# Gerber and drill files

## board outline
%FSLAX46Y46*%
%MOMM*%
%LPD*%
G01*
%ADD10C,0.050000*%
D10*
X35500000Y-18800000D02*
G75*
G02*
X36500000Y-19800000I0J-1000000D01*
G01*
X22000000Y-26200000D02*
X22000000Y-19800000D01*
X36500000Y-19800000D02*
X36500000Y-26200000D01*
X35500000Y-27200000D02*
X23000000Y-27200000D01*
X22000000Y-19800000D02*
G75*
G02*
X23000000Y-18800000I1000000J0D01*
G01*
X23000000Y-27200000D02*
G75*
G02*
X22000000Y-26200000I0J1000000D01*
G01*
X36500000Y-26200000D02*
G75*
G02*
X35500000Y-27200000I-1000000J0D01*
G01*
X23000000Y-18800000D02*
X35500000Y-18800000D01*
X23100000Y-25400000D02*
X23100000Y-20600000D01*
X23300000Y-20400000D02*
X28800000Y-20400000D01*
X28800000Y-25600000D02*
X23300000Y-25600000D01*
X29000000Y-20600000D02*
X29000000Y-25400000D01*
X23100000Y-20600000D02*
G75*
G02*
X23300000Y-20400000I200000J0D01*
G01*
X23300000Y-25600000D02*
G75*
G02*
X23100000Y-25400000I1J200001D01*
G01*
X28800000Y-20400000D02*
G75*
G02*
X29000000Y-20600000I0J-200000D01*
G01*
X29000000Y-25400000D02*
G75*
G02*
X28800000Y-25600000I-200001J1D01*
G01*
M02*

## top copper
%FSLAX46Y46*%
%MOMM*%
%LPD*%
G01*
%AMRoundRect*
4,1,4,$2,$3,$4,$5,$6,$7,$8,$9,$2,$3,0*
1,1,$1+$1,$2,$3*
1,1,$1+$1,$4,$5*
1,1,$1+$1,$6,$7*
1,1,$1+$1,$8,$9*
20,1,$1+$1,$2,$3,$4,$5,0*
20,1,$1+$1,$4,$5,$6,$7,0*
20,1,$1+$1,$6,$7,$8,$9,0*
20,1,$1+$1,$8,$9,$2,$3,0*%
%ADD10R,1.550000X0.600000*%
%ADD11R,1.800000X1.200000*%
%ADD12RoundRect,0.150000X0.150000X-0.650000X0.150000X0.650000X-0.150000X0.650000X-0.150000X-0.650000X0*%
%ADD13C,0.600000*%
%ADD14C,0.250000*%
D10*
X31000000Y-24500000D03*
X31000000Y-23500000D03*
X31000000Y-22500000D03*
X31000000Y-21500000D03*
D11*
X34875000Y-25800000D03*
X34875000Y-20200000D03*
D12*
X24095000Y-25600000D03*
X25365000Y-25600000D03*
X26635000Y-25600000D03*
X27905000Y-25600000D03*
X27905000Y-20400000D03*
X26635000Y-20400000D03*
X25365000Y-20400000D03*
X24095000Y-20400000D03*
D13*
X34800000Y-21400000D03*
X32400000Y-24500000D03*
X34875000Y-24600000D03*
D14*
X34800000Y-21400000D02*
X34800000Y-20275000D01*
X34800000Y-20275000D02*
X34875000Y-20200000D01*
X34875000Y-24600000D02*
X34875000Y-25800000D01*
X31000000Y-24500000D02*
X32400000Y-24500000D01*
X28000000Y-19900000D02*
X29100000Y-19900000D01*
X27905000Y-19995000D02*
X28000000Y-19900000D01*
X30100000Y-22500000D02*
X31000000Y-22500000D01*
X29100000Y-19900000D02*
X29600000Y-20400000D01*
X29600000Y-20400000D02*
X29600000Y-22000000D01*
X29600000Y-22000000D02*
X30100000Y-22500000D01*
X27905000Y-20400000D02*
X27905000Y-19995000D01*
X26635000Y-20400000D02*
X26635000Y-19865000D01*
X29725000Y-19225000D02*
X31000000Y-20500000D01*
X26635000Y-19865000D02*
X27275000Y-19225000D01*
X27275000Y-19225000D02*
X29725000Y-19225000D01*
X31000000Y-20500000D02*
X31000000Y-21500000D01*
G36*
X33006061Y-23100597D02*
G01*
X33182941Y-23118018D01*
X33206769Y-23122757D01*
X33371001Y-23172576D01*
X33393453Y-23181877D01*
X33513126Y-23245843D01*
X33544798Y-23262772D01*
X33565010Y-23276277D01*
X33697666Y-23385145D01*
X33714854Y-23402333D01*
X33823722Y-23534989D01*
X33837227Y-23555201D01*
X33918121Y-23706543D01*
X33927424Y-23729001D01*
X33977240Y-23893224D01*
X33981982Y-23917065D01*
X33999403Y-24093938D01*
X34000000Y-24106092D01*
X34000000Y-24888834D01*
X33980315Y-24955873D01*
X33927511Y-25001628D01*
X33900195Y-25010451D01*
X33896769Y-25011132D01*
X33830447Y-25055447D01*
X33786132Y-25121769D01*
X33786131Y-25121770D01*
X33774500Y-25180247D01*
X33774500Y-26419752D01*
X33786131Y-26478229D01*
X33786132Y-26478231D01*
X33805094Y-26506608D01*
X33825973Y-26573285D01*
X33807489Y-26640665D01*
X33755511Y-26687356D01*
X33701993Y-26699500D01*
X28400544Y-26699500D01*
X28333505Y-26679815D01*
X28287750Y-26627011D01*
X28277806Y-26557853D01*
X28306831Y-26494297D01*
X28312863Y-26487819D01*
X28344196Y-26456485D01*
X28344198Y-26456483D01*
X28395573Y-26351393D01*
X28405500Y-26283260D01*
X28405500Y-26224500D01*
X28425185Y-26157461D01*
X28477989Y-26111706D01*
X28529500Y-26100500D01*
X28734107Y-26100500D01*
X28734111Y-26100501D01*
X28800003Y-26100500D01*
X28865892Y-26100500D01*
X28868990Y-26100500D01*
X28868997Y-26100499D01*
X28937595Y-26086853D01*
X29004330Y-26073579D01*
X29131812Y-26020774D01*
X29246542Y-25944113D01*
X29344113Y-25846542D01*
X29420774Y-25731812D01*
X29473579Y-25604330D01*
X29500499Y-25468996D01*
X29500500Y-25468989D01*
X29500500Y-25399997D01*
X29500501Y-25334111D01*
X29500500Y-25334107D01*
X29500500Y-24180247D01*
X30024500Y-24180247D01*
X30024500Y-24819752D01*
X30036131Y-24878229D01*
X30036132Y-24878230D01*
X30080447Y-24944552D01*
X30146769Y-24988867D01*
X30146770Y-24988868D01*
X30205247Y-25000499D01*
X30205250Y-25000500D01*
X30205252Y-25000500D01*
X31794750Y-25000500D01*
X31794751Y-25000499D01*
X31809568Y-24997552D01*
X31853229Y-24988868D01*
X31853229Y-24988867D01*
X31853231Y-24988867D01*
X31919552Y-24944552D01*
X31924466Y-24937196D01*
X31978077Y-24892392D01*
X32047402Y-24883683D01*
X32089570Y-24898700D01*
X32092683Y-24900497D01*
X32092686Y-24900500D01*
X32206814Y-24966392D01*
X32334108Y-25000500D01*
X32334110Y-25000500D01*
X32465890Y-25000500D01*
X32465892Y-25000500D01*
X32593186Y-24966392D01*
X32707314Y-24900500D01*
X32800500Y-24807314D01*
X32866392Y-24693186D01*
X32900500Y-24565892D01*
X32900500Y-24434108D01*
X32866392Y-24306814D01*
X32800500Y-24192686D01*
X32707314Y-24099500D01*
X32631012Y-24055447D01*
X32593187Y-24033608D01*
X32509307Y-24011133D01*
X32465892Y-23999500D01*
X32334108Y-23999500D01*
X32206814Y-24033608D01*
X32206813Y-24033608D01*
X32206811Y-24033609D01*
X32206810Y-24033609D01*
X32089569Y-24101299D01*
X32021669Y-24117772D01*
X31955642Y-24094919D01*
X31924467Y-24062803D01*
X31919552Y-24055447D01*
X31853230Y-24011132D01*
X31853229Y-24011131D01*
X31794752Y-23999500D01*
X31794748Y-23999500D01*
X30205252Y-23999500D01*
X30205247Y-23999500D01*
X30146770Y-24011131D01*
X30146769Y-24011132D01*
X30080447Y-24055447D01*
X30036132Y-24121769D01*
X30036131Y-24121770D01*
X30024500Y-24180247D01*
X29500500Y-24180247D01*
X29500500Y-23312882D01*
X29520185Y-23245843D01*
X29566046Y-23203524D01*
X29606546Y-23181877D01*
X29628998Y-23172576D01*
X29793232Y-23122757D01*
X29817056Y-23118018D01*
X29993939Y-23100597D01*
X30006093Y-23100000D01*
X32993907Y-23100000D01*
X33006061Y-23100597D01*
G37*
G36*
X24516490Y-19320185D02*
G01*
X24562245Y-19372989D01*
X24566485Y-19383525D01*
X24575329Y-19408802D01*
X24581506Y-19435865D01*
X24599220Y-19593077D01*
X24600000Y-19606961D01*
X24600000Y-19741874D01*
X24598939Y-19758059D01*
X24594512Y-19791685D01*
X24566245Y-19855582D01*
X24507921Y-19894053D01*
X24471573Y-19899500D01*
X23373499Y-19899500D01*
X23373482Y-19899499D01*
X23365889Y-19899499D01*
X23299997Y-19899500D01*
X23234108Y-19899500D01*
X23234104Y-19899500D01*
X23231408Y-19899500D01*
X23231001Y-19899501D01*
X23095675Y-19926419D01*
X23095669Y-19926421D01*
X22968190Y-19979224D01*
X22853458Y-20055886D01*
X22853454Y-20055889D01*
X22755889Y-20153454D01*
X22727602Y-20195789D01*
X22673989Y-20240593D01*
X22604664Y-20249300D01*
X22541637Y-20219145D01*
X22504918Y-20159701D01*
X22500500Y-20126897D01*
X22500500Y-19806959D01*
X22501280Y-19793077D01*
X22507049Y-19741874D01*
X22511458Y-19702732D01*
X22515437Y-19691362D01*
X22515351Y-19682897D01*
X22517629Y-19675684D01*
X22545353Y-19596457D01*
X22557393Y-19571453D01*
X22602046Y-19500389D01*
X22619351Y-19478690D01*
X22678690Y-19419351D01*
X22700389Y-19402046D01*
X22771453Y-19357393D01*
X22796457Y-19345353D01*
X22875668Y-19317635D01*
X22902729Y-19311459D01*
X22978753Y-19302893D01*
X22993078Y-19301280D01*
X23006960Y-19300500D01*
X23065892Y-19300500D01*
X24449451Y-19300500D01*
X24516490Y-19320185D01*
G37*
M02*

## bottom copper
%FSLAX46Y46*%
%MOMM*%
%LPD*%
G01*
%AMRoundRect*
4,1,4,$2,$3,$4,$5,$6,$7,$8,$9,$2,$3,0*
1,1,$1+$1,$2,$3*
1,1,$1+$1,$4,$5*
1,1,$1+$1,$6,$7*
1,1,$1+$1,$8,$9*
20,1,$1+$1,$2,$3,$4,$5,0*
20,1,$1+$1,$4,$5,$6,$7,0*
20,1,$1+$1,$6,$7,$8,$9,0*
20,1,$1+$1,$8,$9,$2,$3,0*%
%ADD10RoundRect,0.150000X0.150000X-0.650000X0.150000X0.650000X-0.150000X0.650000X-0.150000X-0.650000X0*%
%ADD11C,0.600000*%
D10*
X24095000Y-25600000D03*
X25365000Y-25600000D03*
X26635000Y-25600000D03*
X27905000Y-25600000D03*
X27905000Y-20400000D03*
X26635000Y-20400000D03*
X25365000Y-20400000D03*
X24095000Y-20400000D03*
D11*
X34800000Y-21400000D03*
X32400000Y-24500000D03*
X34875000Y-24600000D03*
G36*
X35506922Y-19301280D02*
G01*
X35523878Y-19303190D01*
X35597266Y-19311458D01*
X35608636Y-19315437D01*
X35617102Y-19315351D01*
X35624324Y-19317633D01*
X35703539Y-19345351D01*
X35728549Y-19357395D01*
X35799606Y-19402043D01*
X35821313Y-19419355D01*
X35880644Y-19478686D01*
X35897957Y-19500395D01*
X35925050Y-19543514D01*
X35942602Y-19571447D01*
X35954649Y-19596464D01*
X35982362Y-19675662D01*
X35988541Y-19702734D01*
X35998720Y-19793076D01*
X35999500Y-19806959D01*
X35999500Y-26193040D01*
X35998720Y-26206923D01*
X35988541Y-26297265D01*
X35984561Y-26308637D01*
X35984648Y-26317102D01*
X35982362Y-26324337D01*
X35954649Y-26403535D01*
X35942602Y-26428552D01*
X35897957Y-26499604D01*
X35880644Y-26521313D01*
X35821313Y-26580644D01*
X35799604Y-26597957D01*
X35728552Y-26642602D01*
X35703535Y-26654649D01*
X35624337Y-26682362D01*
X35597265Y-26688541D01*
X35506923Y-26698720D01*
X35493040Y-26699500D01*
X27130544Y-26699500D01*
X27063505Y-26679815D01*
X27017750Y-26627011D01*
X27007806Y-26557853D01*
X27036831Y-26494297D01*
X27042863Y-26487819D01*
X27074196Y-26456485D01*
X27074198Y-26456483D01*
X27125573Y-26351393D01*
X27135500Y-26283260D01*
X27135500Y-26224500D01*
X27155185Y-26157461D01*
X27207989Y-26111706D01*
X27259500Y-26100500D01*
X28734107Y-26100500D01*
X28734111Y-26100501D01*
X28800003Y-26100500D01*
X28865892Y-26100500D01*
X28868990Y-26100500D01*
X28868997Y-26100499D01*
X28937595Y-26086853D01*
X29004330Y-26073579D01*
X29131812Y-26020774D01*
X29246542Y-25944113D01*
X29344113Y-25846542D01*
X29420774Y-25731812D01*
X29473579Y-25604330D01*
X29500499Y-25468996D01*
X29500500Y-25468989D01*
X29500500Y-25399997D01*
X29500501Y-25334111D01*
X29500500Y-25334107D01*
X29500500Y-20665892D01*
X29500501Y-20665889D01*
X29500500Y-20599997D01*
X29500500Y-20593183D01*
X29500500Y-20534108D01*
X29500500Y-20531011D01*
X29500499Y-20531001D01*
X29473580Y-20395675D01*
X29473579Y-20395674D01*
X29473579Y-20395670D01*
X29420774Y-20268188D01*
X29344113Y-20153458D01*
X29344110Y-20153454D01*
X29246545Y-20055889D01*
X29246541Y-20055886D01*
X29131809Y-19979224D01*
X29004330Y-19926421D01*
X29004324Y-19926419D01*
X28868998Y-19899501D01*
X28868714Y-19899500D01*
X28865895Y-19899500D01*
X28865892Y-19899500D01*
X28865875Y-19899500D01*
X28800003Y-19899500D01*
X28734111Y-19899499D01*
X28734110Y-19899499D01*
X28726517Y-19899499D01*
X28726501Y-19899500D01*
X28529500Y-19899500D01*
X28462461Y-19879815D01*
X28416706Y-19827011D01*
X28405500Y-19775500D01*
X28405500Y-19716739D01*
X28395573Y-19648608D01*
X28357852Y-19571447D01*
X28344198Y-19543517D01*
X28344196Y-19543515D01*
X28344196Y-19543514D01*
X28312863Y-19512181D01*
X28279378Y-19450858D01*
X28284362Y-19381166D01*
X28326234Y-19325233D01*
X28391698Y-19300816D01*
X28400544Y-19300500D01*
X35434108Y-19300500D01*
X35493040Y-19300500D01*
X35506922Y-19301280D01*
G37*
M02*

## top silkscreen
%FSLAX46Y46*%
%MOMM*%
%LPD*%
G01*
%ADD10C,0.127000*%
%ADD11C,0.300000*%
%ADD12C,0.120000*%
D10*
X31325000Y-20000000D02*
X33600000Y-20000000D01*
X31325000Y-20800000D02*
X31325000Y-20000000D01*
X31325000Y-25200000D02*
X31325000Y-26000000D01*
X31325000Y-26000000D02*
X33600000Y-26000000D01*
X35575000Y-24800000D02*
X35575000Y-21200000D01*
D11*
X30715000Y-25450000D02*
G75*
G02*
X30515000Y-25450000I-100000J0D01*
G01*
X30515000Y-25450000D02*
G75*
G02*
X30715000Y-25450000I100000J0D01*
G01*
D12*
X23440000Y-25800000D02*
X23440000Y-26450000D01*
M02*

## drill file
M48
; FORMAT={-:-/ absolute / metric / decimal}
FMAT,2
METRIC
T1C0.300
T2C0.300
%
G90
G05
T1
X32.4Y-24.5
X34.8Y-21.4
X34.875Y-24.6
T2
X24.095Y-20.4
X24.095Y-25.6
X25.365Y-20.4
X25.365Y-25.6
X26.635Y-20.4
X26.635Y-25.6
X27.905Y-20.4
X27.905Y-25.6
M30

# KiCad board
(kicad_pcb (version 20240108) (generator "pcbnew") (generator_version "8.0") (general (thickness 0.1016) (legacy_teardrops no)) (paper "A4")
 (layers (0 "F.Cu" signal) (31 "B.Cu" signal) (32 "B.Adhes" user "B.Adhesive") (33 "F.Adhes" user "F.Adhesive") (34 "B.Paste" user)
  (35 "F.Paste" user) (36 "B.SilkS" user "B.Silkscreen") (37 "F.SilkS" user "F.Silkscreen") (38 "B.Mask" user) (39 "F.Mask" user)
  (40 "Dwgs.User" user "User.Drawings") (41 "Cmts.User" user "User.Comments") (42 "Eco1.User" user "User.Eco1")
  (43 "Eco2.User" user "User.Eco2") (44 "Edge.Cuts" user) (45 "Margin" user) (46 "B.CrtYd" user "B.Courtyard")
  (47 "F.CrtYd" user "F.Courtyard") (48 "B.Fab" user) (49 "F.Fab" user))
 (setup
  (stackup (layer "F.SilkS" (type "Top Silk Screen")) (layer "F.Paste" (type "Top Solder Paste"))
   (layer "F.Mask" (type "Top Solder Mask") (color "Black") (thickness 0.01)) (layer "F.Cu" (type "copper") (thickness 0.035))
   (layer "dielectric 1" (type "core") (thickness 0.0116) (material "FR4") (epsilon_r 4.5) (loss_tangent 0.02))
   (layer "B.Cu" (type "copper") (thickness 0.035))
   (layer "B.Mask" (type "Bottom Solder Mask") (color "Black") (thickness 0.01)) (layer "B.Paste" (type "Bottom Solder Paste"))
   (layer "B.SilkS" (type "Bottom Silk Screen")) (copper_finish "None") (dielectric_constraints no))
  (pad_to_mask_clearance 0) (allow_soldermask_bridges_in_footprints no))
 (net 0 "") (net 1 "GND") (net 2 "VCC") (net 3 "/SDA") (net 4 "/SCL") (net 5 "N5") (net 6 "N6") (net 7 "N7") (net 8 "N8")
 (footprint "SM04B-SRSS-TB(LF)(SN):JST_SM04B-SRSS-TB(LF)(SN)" (layer "F.Cu") (at 31 23 90)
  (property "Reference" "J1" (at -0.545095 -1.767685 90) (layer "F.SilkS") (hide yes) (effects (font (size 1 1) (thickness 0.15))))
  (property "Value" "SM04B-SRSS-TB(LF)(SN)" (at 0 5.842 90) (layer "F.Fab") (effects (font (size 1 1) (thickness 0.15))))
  (fp_line (start 3 0.325) (end 3 2.6) (stroke (width 0.127) (type solid)) (layer "F.SilkS"))
  (fp_line (start 2.2 0.325) (end 3 0.325) (stroke (width 0.127) (type solid)) (layer "F.SilkS"))
  (fp_line (start -2.2 0.325) (end -3 0.325) (stroke (width 0.127) (type solid)) (layer "F.SilkS"))
  (fp_line (start -3 0.325) (end -3 2.6) (stroke (width 0.127) (type solid)) (layer "F.SilkS"))
  (fp_line (start -1.8 4.575) (end 1.8 4.575) (stroke (width 0.127) (type solid)) (layer "F.SilkS"))
  (fp_circle (center -2.45 -0.385) (end -2.35 -0.385) (stroke (width 0.3) (type solid)) (fill none) (layer "F.SilkS"))
  (pad "1" smd rect (at -1.5 0 90) (size 0.6 1.55) (layers "F.Cu" "F.Paste" "F.Mask") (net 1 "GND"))
  (pad "2" smd rect (at -0.5 0 90) (size 0.6 1.55) (layers "F.Cu" "F.Paste" "F.Mask") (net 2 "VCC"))
  (pad "3" smd rect (at 0.5 0 90) (size 0.6 1.55) (layers "F.Cu" "F.Paste" "F.Mask") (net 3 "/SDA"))
  (pad "4" smd rect (at 1.5 0 90) (size 0.6 1.55) (layers "F.Cu" "F.Paste" "F.Mask") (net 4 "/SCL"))
  (pad "S1" smd rect (at -2.8 3.875 90) (size 1.2 1.8) (layers "F.Cu" "F.Paste" "F.Mask") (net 1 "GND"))
  (pad "S2" smd rect (at 2.8 3.875 90) (size 1.2 1.8) (layers "F.Cu" "F.Paste" "F.Mask") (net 1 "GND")))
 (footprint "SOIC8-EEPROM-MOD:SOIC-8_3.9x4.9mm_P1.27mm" (layer "F.Cu") (at 26 23 90)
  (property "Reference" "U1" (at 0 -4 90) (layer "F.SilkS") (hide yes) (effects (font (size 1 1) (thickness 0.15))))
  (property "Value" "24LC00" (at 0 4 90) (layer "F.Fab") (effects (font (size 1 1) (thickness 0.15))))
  (fp_line (start -2.8 -2.56) (end -3.45 -2.56) (stroke (width 0.12) (type solid)) (layer "F.SilkS"))
  (fp_line (start -2.4 -2.9) (end 2.4 -2.9) (stroke (width 0.05) (type default)) (layer "Edge.Cuts"))
  (fp_line (start 2.6 -2.7) (end 2.6 2.8) (stroke (width 0.05) (type default)) (layer "Edge.Cuts"))
  (fp_line (start -2.6 2.8) (end -2.6 -2.7) (stroke (width 0.05) (type default)) (layer "Edge.Cuts"))
  (fp_line (start 2.4 3) (end -2.4 3) (stroke (width 0.05) (type default)) (layer "Edge.Cuts"))
  (fp_arc (start 2.4 -2.9) (mid 2.541421 -2.841421) (end 2.6 -2.7) (stroke (width 0.05) (type default)) (layer "Edge.Cuts"))
  (fp_arc (start -2.6 -2.7) (mid -2.541421 -2.841421) (end -2.4 -2.9) (stroke (width 0.05) (type default)) (layer "Edge.Cuts"))
  (fp_arc (start 2.6 2.8) (mid 2.541421 2.941421) (end 2.4 3) (stroke (width 0.05) (type default)) (layer "Edge.Cuts"))
  (fp_arc (start -2.4 3) (mid -2.541421 2.941421) (end -2.6 2.8) (stroke (width 0.05) (type default)) (layer "Edge.Cuts"))
  (pad "1" thru_hole roundrect (at -2.6 -1.905 90) (size 1.6 0.6) (drill 0.3) (layers "*.Cu" "*.Mask") (remove_unused_layers no)
   (roundrect_rratio 0.25) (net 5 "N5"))
  (pad "2" thru_hole roundrect (at -2.6 -0.635 90) (size 1.6 0.6) (drill 0.3) (layers "*.Cu" "*.Mask") (remove_unused_layers no)
   (roundrect_rratio 0.25) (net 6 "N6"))
  (pad "3" thru_hole roundrect (at -2.6 0.635 90) (size 1.6 0.6) (drill 0.3) (layers "*.Cu" "*.Mask") (remove_unused_layers no)
   (roundrect_rratio 0.25) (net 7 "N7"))
  (pad "4" thru_hole roundrect (at -2.6 1.905 90) (size 1.6 0.6) (drill 0.3) (layers "*.Cu" "*.Mask") (remove_unused_layers no)
   (roundrect_rratio 0.25) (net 1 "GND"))
  (pad "5" thru_hole roundrect (at 2.6 1.905 90) (size 1.6 0.6) (drill 0.3) (layers "*.Cu" "*.Mask") (remove_unused_layers no)
   (roundrect_rratio 0.25) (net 3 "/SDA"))
  (pad "6" thru_hole roundrect (at 2.6 0.635 90) (size 1.6 0.6) (drill 0.3) (layers "*.Cu" "*.Mask") (remove_unused_layers no)
   (roundrect_rratio 0.25) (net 4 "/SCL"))
  (pad "7" thru_hole roundrect (at 2.6 -0.635 90) (size 1.6 0.6) (drill 0.3) (layers "*.Cu" "*.Mask") (remove_unused_layers no)
   (roundrect_rratio 0.25) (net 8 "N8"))
  (pad "8" thru_hole roundrect (at 2.6 -1.905 90) (size 1.6 0.6) (drill 0.3) (layers "*.Cu" "*.Mask") (remove_unused_layers no)
   (roundrect_rratio 0.25) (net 2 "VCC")))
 (gr_arc (start 35.5 18.8) (mid 36.207107 19.092893) (end 36.5 19.8) (stroke (width 0.05) (type default)) (layer "Edge.Cuts"))
 (gr_line (start 22 26.2) (end 22 19.8) (stroke (width 0.05) (type default)) (layer "Edge.Cuts"))
 (gr_line (start 36.5 19.8) (end 36.5 26.2) (stroke (width 0.05) (type default)) (layer "Edge.Cuts"))
 (gr_line (start 35.5 27.2) (end 23 27.2) (stroke (width 0.05) (type default)) (layer "Edge.Cuts"))
 (gr_arc (start 22 19.8) (mid 22.292893 19.092893) (end 23 18.8) (stroke (width 0.05) (type default)) (layer "Edge.Cuts"))
 (gr_arc (start 23 27.2) (mid 22.292893 26.907107) (end 22 26.2) (stroke (width 0.05) (type default)) (layer "Edge.Cuts"))
 (gr_arc (start 36.5 26.2) (mid 36.207107 26.907107) (end 35.5 27.2) (stroke (width 0.05) (type default)) (layer "Edge.Cuts"))
 (gr_line (start 23 18.8) (end 35.5 18.8) (stroke (width 0.05) (type default)) (layer "Edge.Cuts"))
 (segment (start 34.8 21.4) (end 34.8 20.275) (width 0.25) (layer "F.Cu") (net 1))
 (segment (start 34.8 20.275) (end 34.875 20.2) (width 0.25) (layer "F.Cu") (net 1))
 (segment (start 34.875 24.6) (end 34.875 25.8) (width 0.25) (layer "F.Cu") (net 1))
 (segment (start 31 24.5) (end 32.4 24.5) (width 0.25) (layer "F.Cu") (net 1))
 (via (at 34.8 21.4) (size 0.6) (drill 0.3) (layers "F.Cu" "B.Cu") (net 1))
 (via (at 32.4 24.5) (size 0.6) (drill 0.3) (layers "F.Cu" "B.Cu") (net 1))
 (via (at 34.875 24.6) (size 0.6) (drill 0.3) (layers "F.Cu" "B.Cu") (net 1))
 (segment (start 28 19.9) (end 29.1 19.9) (width 0.25) (layer "F.Cu") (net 3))
 (segment (start 27.905 19.995) (end 28 19.9) (width 0.25) (layer "F.Cu") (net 3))
 (segment (start 30.1 22.5) (end 31 22.5) (width 0.25) (layer "F.Cu") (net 3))
 (segment (start 29.1 19.9) (end 29.6 20.4) (width 0.25) (layer "F.Cu") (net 3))
 (segment (start 29.6 20.4) (end 29.6 22) (width 0.25) (layer "F.Cu") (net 3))
 (segment (start 29.6 22) (end 30.1 22.5) (width 0.25) (layer "F.Cu") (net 3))
 (segment (start 27.905 20.4) (end 27.905 19.995) (width 0.25) (layer "F.Cu") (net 3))
 (segment (start 26.635 20.4) (end 26.635 19.865) (width 0.25) (layer "F.Cu") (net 4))
 (segment (start 29.725 19.225) (end 31 20.5) (width 0.25) (layer "F.Cu") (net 4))
 (segment (start 26.635 19.865) (end 27.275 19.225) (width 0.25) (layer "F.Cu") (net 4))
 (segment (start 27.275 19.225) (end 29.725 19.225) (width 0.25) (layer "F.Cu") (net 4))
 (segment (start 31 20.5) (end 31 21.5) (width 0.25) (layer "F.Cu") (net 4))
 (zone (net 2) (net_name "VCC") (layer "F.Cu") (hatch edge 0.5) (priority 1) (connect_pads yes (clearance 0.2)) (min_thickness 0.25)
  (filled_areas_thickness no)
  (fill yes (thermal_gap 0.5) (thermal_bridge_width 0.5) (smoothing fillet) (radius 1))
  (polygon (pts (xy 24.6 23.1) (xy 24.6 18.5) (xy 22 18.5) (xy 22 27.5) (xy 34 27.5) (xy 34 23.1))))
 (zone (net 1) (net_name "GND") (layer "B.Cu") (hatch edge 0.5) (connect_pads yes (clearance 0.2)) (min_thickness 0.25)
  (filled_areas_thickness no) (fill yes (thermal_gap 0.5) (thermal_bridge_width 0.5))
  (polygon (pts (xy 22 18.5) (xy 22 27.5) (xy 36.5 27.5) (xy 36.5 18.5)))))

